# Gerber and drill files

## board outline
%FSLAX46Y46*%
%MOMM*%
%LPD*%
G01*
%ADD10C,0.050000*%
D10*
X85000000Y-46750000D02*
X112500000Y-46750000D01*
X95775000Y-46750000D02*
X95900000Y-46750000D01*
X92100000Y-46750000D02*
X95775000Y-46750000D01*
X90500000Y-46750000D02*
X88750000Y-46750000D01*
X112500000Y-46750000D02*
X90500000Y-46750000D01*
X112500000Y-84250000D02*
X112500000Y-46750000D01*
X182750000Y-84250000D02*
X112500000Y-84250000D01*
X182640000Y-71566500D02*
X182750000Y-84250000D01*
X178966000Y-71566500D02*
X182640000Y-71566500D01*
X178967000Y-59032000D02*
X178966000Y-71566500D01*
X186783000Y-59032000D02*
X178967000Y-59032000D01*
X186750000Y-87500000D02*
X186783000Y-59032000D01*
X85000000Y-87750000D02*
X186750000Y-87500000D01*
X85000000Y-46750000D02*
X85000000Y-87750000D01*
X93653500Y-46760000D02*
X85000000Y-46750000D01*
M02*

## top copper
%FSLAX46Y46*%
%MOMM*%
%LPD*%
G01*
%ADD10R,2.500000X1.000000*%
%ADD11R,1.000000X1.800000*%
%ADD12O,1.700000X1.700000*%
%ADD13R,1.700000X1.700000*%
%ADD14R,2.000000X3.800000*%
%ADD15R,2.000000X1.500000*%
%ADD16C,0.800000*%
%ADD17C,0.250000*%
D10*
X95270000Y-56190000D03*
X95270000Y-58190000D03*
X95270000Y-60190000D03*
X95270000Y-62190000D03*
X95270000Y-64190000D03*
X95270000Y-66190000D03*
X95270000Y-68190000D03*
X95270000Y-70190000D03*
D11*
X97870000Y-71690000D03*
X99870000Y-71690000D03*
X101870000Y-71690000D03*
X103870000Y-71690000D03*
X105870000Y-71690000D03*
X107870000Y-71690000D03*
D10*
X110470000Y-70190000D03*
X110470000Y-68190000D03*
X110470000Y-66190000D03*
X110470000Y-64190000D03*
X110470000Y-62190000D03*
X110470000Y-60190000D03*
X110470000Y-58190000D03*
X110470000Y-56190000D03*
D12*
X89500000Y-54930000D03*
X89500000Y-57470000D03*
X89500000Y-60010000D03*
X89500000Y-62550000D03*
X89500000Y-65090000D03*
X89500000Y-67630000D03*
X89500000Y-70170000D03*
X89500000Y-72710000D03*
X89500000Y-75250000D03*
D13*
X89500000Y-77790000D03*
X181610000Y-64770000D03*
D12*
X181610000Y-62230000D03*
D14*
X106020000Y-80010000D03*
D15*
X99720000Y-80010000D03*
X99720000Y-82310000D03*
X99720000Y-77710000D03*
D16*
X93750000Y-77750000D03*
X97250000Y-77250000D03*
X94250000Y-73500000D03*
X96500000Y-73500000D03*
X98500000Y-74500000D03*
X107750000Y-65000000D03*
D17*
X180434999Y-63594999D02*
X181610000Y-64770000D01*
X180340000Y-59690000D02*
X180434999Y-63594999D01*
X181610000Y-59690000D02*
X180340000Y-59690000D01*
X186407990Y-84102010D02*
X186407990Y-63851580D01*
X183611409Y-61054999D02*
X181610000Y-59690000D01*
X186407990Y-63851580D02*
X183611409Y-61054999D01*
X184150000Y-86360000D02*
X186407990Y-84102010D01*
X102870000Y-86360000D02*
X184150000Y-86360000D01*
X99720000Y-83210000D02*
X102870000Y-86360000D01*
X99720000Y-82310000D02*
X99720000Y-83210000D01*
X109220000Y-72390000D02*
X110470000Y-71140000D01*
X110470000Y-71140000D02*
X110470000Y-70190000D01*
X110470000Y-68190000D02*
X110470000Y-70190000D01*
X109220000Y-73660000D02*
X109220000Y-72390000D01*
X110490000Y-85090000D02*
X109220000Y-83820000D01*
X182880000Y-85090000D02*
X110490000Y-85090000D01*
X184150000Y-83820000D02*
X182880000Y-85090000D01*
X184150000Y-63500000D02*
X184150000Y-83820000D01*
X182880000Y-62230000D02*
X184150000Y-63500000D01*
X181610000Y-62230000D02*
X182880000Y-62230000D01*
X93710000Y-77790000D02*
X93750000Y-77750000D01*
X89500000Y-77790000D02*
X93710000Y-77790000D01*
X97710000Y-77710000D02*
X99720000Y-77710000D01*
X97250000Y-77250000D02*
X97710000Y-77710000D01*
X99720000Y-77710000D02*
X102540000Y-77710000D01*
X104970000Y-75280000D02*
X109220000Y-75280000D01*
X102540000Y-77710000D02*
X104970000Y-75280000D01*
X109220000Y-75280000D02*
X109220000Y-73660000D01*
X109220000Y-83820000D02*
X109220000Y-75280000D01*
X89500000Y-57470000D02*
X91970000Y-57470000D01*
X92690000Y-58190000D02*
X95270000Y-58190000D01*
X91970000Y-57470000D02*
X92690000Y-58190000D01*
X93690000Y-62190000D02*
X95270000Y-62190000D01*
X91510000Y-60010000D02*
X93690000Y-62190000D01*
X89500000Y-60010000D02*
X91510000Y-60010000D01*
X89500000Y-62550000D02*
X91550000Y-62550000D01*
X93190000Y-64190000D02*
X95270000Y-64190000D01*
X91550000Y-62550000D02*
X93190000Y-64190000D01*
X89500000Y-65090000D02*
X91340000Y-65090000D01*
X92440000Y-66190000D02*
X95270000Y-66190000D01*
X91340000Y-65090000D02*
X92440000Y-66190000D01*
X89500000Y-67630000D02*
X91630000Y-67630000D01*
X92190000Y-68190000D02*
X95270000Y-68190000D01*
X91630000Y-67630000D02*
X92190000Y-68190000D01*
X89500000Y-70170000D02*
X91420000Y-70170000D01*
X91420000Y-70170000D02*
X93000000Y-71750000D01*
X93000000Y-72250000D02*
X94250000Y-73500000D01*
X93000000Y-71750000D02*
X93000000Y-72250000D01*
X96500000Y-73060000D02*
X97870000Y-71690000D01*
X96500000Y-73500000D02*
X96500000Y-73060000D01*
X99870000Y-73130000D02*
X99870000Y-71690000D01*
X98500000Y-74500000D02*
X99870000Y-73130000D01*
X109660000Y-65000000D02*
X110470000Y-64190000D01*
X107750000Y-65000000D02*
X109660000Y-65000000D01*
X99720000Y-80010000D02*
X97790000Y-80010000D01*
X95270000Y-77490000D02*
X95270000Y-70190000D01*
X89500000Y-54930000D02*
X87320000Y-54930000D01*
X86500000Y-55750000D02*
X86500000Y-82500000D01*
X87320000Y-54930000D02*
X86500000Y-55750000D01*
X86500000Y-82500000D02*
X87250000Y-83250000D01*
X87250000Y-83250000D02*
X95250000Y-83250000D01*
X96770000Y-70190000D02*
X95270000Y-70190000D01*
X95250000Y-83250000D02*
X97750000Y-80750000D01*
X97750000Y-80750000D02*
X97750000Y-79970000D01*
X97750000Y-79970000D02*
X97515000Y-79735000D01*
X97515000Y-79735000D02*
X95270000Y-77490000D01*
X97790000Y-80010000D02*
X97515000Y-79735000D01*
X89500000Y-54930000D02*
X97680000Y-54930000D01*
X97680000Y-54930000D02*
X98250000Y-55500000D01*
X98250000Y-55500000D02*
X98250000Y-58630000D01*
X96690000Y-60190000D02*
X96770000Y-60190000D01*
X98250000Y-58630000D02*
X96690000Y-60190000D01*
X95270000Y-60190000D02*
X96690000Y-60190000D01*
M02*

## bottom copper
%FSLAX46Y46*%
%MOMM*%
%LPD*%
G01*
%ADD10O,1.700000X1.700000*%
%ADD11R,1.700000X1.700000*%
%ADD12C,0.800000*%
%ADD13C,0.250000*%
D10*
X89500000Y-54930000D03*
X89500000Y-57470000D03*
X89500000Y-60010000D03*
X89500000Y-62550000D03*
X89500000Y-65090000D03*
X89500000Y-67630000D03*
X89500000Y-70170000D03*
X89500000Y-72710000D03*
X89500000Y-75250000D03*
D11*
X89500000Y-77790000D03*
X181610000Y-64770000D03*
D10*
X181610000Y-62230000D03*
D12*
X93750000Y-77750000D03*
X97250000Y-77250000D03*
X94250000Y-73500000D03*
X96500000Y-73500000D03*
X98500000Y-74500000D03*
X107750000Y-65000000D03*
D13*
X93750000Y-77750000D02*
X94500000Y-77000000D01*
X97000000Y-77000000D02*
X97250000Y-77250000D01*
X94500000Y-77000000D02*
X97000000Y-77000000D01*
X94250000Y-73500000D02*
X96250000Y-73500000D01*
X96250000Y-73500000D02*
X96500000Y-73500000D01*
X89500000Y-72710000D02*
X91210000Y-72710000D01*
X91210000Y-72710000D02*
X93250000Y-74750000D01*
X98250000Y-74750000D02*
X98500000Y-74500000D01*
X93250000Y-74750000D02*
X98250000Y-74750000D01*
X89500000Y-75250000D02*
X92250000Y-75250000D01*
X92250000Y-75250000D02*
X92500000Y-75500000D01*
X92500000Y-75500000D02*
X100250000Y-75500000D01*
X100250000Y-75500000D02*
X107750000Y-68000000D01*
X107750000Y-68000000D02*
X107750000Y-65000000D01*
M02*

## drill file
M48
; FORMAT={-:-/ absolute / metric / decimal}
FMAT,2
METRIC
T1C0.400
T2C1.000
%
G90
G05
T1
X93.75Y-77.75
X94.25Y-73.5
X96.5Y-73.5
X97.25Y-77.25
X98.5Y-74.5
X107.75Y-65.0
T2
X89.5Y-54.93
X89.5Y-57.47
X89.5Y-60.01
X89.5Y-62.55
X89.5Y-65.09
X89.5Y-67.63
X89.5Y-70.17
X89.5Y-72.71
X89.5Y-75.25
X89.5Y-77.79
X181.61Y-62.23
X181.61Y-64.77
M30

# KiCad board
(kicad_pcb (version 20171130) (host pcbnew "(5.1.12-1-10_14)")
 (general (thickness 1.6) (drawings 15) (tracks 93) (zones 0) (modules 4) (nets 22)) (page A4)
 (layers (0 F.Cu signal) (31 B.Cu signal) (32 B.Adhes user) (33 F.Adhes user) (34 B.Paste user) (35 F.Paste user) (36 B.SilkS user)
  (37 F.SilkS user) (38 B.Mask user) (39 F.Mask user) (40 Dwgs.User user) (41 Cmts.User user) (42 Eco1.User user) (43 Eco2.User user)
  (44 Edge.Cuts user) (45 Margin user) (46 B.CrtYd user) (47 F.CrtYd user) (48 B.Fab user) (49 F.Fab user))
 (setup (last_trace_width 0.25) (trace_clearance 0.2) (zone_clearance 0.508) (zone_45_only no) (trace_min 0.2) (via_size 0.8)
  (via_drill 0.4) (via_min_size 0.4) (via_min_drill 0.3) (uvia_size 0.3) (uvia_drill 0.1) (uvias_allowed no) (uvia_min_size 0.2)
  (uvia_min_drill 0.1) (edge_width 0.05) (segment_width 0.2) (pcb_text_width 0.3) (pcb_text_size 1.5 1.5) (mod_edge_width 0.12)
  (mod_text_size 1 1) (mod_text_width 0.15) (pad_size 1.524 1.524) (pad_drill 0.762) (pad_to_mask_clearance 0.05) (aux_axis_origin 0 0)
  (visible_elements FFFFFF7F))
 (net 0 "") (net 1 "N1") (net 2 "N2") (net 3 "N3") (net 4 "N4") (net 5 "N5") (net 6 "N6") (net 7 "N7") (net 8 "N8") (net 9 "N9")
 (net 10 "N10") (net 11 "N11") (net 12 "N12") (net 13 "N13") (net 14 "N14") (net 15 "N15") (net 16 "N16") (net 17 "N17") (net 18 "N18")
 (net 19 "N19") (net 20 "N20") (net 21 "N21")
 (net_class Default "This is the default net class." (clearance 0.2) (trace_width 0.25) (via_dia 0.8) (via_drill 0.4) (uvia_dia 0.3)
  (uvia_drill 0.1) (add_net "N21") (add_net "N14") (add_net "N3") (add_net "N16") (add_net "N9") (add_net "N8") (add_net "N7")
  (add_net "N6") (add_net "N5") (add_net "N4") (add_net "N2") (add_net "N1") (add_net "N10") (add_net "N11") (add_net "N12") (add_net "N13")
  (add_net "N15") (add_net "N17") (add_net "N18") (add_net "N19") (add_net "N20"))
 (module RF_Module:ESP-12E (layer F.Cu) (at 102.87 59.69)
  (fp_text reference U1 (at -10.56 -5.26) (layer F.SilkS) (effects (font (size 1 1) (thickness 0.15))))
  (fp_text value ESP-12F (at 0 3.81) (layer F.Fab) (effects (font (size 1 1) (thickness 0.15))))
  (pad 1 smd rect (at -7.6 -3.5) (size 2.5 1) (layers F.Cu F.Paste F.Mask) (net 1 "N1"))
  (pad 2 smd rect (at -7.6 -1.5) (size 2.5 1) (layers F.Cu F.Paste F.Mask) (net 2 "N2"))
  (pad 3 smd rect (at -7.6 0.5) (size 2.5 1) (layers F.Cu F.Paste F.Mask) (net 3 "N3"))
  (pad 4 smd rect (at -7.6 2.5) (size 2.5 1) (layers F.Cu F.Paste F.Mask) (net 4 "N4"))
  (pad 5 smd rect (at -7.6 4.5) (size 2.5 1) (layers F.Cu F.Paste F.Mask) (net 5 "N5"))
  (pad 6 smd rect (at -7.6 6.5) (size 2.5 1) (layers F.Cu F.Paste F.Mask) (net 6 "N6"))
  (pad 7 smd rect (at -7.6 8.5) (size 2.5 1) (layers F.Cu F.Paste F.Mask) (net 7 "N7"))
  (pad 8 smd rect (at -7.6 10.5) (size 2.5 1) (layers F.Cu F.Paste F.Mask) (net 3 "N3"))
  (pad 9 smd rect (at -5 12) (size 1 1.8) (layers F.Cu F.Paste F.Mask) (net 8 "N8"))
  (pad 10 smd rect (at -3 12) (size 1 1.8) (layers F.Cu F.Paste F.Mask) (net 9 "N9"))
  (pad 11 smd rect (at -1 12) (size 1 1.8) (layers F.Cu F.Paste F.Mask) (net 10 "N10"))
  (pad 12 smd rect (at 1 12) (size 1 1.8) (layers F.Cu F.Paste F.Mask) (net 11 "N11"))
  (pad 13 smd rect (at 3 12) (size 1 1.8) (layers F.Cu F.Paste F.Mask) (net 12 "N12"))
  (pad 14 smd rect (at 5 12) (size 1 1.8) (layers F.Cu F.Paste F.Mask) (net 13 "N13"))
  (pad 15 smd rect (at 7.6 10.5) (size 2.5 1) (layers F.Cu F.Paste F.Mask) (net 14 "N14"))
  (pad 16 smd rect (at 7.6 8.5) (size 2.5 1) (layers F.Cu F.Paste F.Mask) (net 14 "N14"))
  (pad 17 smd rect (at 7.6 6.5) (size 2.5 1) (layers F.Cu F.Paste F.Mask) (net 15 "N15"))
  (pad 18 smd rect (at 7.6 4.5) (size 2.5 1) (layers F.Cu F.Paste F.Mask) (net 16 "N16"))
  (pad 19 smd rect (at 7.6 2.5) (size 2.5 1) (layers F.Cu F.Paste F.Mask) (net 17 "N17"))
  (pad 20 smd rect (at 7.6 0.5) (size 2.5 1) (layers F.Cu F.Paste F.Mask) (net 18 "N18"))
  (pad 21 smd rect (at 7.6 -1.5) (size 2.5 1) (layers F.Cu F.Paste F.Mask) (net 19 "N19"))
  (pad 22 smd rect (at 7.6 -3.5) (size 2.5 1) (layers F.Cu F.Paste F.Mask) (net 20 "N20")))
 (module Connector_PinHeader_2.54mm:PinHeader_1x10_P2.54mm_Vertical (layer F.Cu) (at 89.5 77.79 180)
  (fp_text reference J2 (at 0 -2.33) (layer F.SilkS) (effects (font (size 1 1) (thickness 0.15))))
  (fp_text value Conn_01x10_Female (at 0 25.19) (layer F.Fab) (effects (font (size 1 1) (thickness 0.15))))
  (pad 10 thru_hole oval (at 0 22.86 180) (size 1.7 1.7) (drill 1) (layers *.Cu *.Mask) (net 3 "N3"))
  (pad 9 thru_hole oval (at 0 20.32 180) (size 1.7 1.7) (drill 1) (layers *.Cu *.Mask) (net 2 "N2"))
  (pad 8 thru_hole oval (at 0 17.78 180) (size 1.7 1.7) (drill 1) (layers *.Cu *.Mask) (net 4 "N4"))
  (pad 7 thru_hole oval (at 0 15.24 180) (size 1.7 1.7) (drill 1) (layers *.Cu *.Mask) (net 5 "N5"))
  (pad 6 thru_hole oval (at 0 12.7 180) (size 1.7 1.7) (drill 1) (layers *.Cu *.Mask) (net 6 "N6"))
  (pad 5 thru_hole oval (at 0 10.16 180) (size 1.7 1.7) (drill 1) (layers *.Cu *.Mask) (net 7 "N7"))
  (pad 4 thru_hole oval (at 0 7.62 180) (size 1.7 1.7) (drill 1) (layers *.Cu *.Mask) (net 8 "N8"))
  (pad 3 thru_hole oval (at 0 5.08 180) (size 1.7 1.7) (drill 1) (layers *.Cu *.Mask) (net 9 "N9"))
  (pad 2 thru_hole oval (at 0 2.54 180) (size 1.7 1.7) (drill 1) (layers *.Cu *.Mask) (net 16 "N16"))
  (pad 1 thru_hole rect (at 0 0 180) (size 1.7 1.7) (drill 1) (layers *.Cu *.Mask) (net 14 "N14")))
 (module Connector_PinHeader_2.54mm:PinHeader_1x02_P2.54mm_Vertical (layer F.Cu) (at 181.61 64.77 180)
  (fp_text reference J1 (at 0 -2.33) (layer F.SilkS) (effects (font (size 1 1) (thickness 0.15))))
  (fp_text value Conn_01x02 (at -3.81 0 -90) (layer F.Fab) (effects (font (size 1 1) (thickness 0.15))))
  (pad 1 thru_hole rect (at 0 0 180) (size 1.7 1.7) (drill 1) (layers *.Cu *.Mask) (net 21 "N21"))
  (pad 2 thru_hole oval (at 0 2.54 180) (size 1.7 1.7) (drill 1) (layers *.Cu *.Mask) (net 14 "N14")))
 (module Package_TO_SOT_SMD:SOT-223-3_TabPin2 (layer F.Cu) (at 102.87 80.01)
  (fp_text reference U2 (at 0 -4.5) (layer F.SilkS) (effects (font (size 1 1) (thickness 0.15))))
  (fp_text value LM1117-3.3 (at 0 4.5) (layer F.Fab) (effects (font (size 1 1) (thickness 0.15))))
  (pad 2 smd rect (at 3.15 0) (size 2 3.8) (layers F.Cu F.Paste F.Mask) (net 3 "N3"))
  (pad 2 smd rect (at -3.15 0) (size 2 1.5) (layers F.Cu F.Paste F.Mask) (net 3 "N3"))
  (pad 3 smd rect (at -3.15 2.3) (size 2 1.5) (layers F.Cu F.Paste F.Mask) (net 21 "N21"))
  (pad 1 smd rect (at -3.15 -2.3) (size 2 1.5) (layers F.Cu F.Paste F.Mask) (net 14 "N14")))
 (gr_line (start 85 46.75) (end 112.5 46.75) (layer Edge.Cuts) (width 0.05))
 (gr_line (start 95.775 46.75) (end 95.9 46.75) (layer Edge.Cuts) (width 0.05))
 (gr_line (start 92.1 46.75) (end 95.775 46.75) (layer Edge.Cuts) (width 0.05))
 (gr_line (start 90.5 46.75) (end 88.75 46.75) (layer Edge.Cuts) (width 0.05))
 (gr_line (start 112.5 46.75) (end 90.5 46.75) (layer Edge.Cuts) (width 0.05))
 (gr_line (start 112.5 84.25) (end 112.5 46.75) (layer Edge.Cuts) (width 0.05))
 (gr_line (start 182.75 84.25) (end 112.5 84.25) (layer Edge.Cuts) (width 0.05))
 (gr_line (start 182.64 71.5665) (end 182.75 84.25) (layer Edge.Cuts) (width 0.05))
 (gr_line (start 178.966 71.5665) (end 182.64 71.5665) (layer Edge.Cuts) (width 0.05))
 (gr_line (start 178.967 59.032) (end 178.966 71.5665) (layer Edge.Cuts) (width 0.05))
 (gr_line (start 186.783 59.032) (end 178.967 59.032) (layer Edge.Cuts) (width 0.05))
 (gr_line (start 186.75 87.5) (end 186.783 59.032) (layer Edge.Cuts) (width 0.05))
 (gr_line (start 85 87.75) (end 186.75 87.5) (layer Edge.Cuts) (width 0.05))
 (gr_line (start 85 46.75) (end 85 87.75) (layer Edge.Cuts) (width 0.05))
 (gr_line (start 93.6535 46.76) (end 85 46.75) (layer Edge.Cuts) (width 0.05))
 (segment (start 180.434999 63.594999) (end 181.61 64.77) (width 0.25) (layer F.Cu) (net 21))
 (segment (start 180.34 59.69) (end 180.434999 63.594999) (width 0.25) (layer F.Cu) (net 21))
 (segment (start 181.61 59.69) (end 180.34 59.69) (width 0.25) (layer F.Cu) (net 21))
 (segment (start 186.40799 84.10201) (end 186.40799 63.85158) (width 0.25) (layer F.Cu) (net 21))
 (segment (start 183.611409 61.054999) (end 181.61 59.69) (width 0.25) (layer F.Cu) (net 21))
 (segment (start 186.40799 63.85158) (end 183.611409 61.054999) (width 0.25) (layer F.Cu) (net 21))
 (segment (start 184.15 86.36) (end 186.40799 84.10201) (width 0.25) (layer F.Cu) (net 21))
 (segment (start 102.87 86.36) (end 184.15 86.36) (width 0.25) (layer F.Cu) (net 21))
 (segment (start 99.72 83.21) (end 102.87 86.36) (width 0.25) (layer F.Cu) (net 21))
 (segment (start 99.72 82.31) (end 99.72 83.21) (width 0.25) (layer F.Cu) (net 21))
 (segment (start 109.22 72.39) (end 110.47 71.14) (width 0.25) (layer F.Cu) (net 14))
 (segment (start 110.47 71.14) (end 110.47 70.19) (width 0.25) (layer F.Cu) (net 14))
 (segment (start 110.47 68.19) (end 110.47 70.19) (width 0.25) (layer F.Cu) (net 14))
 (segment (start 109.22 73.66) (end 109.22 72.39) (width 0.25) (layer F.Cu) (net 14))
 (segment (start 110.49 85.09) (end 109.22 83.82) (width 0.25) (layer F.Cu) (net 14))
 (segment (start 182.88 85.09) (end 110.49 85.09) (width 0.25) (layer F.Cu) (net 14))
 (segment (start 184.15 83.82) (end 182.88 85.09) (width 0.25) (layer F.Cu) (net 14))
 (segment (start 184.15 63.5) (end 184.15 83.82) (width 0.25) (layer F.Cu) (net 14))
 (segment (start 182.88 62.23) (end 184.15 63.5) (width 0.25) (layer F.Cu) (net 14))
 (segment (start 181.61 62.23) (end 182.88 62.23) (width 0.25) (layer F.Cu) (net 14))
 (segment (start 93.71 77.79) (end 93.75 77.75) (width 0.25) (layer F.Cu) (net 14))
 (via (at 93.75 77.75) (size 0.8) (drill 0.4) (layers F.Cu B.Cu) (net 14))
 (segment (start 89.5 77.79) (end 93.71 77.79) (width 0.25) (layer F.Cu) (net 14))
 (segment (start 93.75 77.75) (end 94.5 77) (width 0.25) (layer B.Cu) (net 14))
 (via (at 97.25 77.25) (size 0.8) (drill 0.4) (layers F.Cu B.Cu) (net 14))
 (segment (start 97 77) (end 97.25 77.25) (width 0.25) (layer B.Cu) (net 14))
 (segment (start 94.5 77) (end 97 77) (width 0.25) (layer B.Cu) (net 14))
 (segment (start 97.71 77.71) (end 99.72 77.71) (width 0.25) (layer F.Cu) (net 14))
 (segment (start 97.25 77.25) (end 97.71 77.71) (width 0.25) (layer F.Cu) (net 14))
 (segment (start 99.72 77.71) (end 102.54 77.71) (width 0.25) (layer F.Cu) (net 14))
 (segment (start 104.97 75.28) (end 109.22 75.28) (width 0.25) (layer F.Cu) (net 14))
 (segment (start 102.54 77.71) (end 104.97 75.28) (width 0.25) (layer F.Cu) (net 14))
 (segment (start 109.22 75.28) (end 109.22 73.66) (width 0.25) (layer F.Cu) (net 14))
 (segment (start 109.22 83.82) (end 109.22 75.28) (width 0.25) (layer F.Cu) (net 14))
 (segment (start 89.5 57.47) (end 91.97 57.47) (width 0.25) (layer F.Cu) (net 2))
 (segment (start 92.69 58.19) (end 95.27 58.19) (width 0.25) (layer F.Cu) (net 2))
 (segment (start 91.97 57.47) (end 92.69 58.19) (width 0.25) (layer F.Cu) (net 2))
 (segment (start 93.69 62.19) (end 95.27 62.19) (width 0.25) (layer F.Cu) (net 4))
 (segment (start 91.51 60.01) (end 93.69 62.19) (width 0.25) (layer F.Cu) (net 4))
 (segment (start 89.5 60.01) (end 91.51 60.01) (width 0.25) (layer F.Cu) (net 4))
 (segment (start 89.5 62.55) (end 91.55 62.55) (width 0.25) (layer F.Cu) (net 5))
 (segment (start 93.19 64.19) (end 95.27 64.19) (width 0.25) (layer F.Cu) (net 5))
 (segment (start 91.55 62.55) (end 93.19 64.19) (width 0.25) (layer F.Cu) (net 5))
 (segment (start 89.5 65.09) (end 91.34 65.09) (width 0.25) (layer F.Cu) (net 6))
 (segment (start 92.44 66.19) (end 95.27 66.19) (width 0.25) (layer F.Cu) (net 6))
 (segment (start 91.34 65.09) (end 92.44 66.19) (width 0.25) (layer F.Cu) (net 6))
 (segment (start 89.5 67.63) (end 91.63 67.63) (width 0.25) (layer F.Cu) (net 7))
 (segment (start 92.19 68.19) (end 95.27 68.19) (width 0.25) (layer F.Cu) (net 7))
 (segment (start 91.63 67.63) (end 92.19 68.19) (width 0.25) (layer F.Cu) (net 7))
 (segment (start 89.5 70.17) (end 91.42 70.17) (width 0.25) (layer F.Cu) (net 8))
 (segment (start 91.42 70.17) (end 93 71.75) (width 0.25) (layer F.Cu) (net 8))
 (via (at 94.25 73.5) (size 0.8) (drill 0.4) (layers F.Cu B.Cu) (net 8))
 (segment (start 93 72.25) (end 94.25 73.5) (width 0.25) (layer F.Cu) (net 8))
 (segment (start 93 71.75) (end 93 72.25) (width 0.25) (layer F.Cu) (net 8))
 (segment (start 94.25 73.5) (end 96.25 73.5) (width 0.25) (layer B.Cu) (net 8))
 (via (at 96.5 73.5) (size 0.8) (drill 0.4) (layers F.Cu B.Cu) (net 8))
 (segment (start 96.25 73.5) (end 96.5 73.5) (width 0.25) (layer B.Cu) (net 8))
 (segment (start 96.5 73.06) (end 97.87 71.69) (width 0.25) (layer F.Cu) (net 8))
 (segment (start 96.5 73.5) (end 96.5 73.06) (width 0.25) (layer F.Cu) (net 8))
 (segment (start 89.5 72.71) (end 91.21 72.71) (width 0.25) (layer B.Cu) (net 9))
 (segment (start 91.21 72.71) (end 93.25 74.75) (width 0.25) (layer B.Cu) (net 9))
 (via (at 98.5 74.5) (size 0.8) (drill 0.4) (layers F.Cu B.Cu) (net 9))
 (segment (start 98.25 74.75) (end 98.5 74.5) (width 0.25) (layer B.Cu) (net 9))
 (segment (start 93.25 74.75) (end 98.25 74.75) (width 0.25) (layer B.Cu) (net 9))
 (segment (start 99.87 73.13) (end 99.87 71.69) (width 0.25) (layer F.Cu) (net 9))
 (segment (start 98.5 74.5) (end 99.87 73.13) (width 0.25) (layer F.Cu) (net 9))
 (segment (start 89.5 75.25) (end 92.25 75.25) (width 0.25) (layer B.Cu) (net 16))
 (segment (start 92.25 75.25) (end 92.5 75.5) (width 0.25) (layer B.Cu) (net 16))
 (segment (start 92.5 75.5) (end 100.25 75.5) (width 0.25) (layer B.Cu) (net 16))
 (segment (start 100.25 75.5) (end 107.75 68) (width 0.25) (layer B.Cu) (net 16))
 (via (at 107.75 65) (size 0.8) (drill 0.4) (layers F.Cu B.Cu) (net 16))
 (segment (start 107.75 68) (end 107.75 65) (width 0.25) (layer B.Cu) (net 16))
 (segment (start 109.66 65) (end 110.47 64.19) (width 0.25) (layer F.Cu) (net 16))
 (segment (start 107.75 65) (end 109.66 65) (width 0.25) (layer F.Cu) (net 16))
 (segment (start 99.72 80.01) (end 97.79 80.01) (width 0.25) (layer F.Cu) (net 3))
 (segment (start 95.27 77.49) (end 95.27 70.19) (width 0.25) (layer F.Cu) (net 3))
 (segment (start 89.5 54.93) (end 87.32 54.93) (width 0.25) (layer F.Cu) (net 3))
 (segment (start 86.5 55.75) (end 86.5 82.5) (width 0.25) (layer F.Cu) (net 3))
 (segment (start 87.32 54.93) (end 86.5 55.75) (width 0.25) (layer F.Cu) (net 3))
 (segment (start 86.5 82.5) (end 87.25 83.25) (width 0.25) (layer F.Cu) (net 3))
 (segment (start 87.25 83.25) (end 95.25 83.25) (width 0.25) (layer F.Cu) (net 3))
 (segment (start 96.77 70.19) (end 95.27 70.19) (width 0.25) (layer F.Cu) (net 3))
 (segment (start 95.25 83.25) (end 97.75 80.75) (width 0.25) (layer F.Cu) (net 3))
 (segment (start 97.75 80.75) (end 97.75 79.97) (width 0.25) (layer F.Cu) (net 3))
 (segment (start 97.75 79.97) (end 97.515 79.735) (width 0.25) (layer F.Cu) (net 3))
 (segment (start 97.515 79.735) (end 95.27 77.49) (width 0.25) (layer F.Cu) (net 3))
 (segment (start 97.79 80.01) (end 97.515 79.735) (width 0.25) (layer F.Cu) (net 3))
 (segment (start 89.5 54.93) (end 97.68 54.93) (width 0.25) (layer F.Cu) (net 3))
 (segment (start 97.68 54.93) (end 98.25 55.5) (width 0.25) (layer F.Cu) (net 3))
 (segment (start 98.25 55.5) (end 98.25 58.63) (width 0.25) (layer F.Cu) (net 3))
 (segment (start 96.69 60.19) (end 96.77 60.19) (width 0.25) (layer F.Cu) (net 3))
 (segment (start 98.25 58.63) (end 96.69 60.19) (width 0.25) (layer F.Cu) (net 3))
 (segment (start 95.27 60.19) (end 96.69 60.19) (width 0.25) (layer F.Cu) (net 3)))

